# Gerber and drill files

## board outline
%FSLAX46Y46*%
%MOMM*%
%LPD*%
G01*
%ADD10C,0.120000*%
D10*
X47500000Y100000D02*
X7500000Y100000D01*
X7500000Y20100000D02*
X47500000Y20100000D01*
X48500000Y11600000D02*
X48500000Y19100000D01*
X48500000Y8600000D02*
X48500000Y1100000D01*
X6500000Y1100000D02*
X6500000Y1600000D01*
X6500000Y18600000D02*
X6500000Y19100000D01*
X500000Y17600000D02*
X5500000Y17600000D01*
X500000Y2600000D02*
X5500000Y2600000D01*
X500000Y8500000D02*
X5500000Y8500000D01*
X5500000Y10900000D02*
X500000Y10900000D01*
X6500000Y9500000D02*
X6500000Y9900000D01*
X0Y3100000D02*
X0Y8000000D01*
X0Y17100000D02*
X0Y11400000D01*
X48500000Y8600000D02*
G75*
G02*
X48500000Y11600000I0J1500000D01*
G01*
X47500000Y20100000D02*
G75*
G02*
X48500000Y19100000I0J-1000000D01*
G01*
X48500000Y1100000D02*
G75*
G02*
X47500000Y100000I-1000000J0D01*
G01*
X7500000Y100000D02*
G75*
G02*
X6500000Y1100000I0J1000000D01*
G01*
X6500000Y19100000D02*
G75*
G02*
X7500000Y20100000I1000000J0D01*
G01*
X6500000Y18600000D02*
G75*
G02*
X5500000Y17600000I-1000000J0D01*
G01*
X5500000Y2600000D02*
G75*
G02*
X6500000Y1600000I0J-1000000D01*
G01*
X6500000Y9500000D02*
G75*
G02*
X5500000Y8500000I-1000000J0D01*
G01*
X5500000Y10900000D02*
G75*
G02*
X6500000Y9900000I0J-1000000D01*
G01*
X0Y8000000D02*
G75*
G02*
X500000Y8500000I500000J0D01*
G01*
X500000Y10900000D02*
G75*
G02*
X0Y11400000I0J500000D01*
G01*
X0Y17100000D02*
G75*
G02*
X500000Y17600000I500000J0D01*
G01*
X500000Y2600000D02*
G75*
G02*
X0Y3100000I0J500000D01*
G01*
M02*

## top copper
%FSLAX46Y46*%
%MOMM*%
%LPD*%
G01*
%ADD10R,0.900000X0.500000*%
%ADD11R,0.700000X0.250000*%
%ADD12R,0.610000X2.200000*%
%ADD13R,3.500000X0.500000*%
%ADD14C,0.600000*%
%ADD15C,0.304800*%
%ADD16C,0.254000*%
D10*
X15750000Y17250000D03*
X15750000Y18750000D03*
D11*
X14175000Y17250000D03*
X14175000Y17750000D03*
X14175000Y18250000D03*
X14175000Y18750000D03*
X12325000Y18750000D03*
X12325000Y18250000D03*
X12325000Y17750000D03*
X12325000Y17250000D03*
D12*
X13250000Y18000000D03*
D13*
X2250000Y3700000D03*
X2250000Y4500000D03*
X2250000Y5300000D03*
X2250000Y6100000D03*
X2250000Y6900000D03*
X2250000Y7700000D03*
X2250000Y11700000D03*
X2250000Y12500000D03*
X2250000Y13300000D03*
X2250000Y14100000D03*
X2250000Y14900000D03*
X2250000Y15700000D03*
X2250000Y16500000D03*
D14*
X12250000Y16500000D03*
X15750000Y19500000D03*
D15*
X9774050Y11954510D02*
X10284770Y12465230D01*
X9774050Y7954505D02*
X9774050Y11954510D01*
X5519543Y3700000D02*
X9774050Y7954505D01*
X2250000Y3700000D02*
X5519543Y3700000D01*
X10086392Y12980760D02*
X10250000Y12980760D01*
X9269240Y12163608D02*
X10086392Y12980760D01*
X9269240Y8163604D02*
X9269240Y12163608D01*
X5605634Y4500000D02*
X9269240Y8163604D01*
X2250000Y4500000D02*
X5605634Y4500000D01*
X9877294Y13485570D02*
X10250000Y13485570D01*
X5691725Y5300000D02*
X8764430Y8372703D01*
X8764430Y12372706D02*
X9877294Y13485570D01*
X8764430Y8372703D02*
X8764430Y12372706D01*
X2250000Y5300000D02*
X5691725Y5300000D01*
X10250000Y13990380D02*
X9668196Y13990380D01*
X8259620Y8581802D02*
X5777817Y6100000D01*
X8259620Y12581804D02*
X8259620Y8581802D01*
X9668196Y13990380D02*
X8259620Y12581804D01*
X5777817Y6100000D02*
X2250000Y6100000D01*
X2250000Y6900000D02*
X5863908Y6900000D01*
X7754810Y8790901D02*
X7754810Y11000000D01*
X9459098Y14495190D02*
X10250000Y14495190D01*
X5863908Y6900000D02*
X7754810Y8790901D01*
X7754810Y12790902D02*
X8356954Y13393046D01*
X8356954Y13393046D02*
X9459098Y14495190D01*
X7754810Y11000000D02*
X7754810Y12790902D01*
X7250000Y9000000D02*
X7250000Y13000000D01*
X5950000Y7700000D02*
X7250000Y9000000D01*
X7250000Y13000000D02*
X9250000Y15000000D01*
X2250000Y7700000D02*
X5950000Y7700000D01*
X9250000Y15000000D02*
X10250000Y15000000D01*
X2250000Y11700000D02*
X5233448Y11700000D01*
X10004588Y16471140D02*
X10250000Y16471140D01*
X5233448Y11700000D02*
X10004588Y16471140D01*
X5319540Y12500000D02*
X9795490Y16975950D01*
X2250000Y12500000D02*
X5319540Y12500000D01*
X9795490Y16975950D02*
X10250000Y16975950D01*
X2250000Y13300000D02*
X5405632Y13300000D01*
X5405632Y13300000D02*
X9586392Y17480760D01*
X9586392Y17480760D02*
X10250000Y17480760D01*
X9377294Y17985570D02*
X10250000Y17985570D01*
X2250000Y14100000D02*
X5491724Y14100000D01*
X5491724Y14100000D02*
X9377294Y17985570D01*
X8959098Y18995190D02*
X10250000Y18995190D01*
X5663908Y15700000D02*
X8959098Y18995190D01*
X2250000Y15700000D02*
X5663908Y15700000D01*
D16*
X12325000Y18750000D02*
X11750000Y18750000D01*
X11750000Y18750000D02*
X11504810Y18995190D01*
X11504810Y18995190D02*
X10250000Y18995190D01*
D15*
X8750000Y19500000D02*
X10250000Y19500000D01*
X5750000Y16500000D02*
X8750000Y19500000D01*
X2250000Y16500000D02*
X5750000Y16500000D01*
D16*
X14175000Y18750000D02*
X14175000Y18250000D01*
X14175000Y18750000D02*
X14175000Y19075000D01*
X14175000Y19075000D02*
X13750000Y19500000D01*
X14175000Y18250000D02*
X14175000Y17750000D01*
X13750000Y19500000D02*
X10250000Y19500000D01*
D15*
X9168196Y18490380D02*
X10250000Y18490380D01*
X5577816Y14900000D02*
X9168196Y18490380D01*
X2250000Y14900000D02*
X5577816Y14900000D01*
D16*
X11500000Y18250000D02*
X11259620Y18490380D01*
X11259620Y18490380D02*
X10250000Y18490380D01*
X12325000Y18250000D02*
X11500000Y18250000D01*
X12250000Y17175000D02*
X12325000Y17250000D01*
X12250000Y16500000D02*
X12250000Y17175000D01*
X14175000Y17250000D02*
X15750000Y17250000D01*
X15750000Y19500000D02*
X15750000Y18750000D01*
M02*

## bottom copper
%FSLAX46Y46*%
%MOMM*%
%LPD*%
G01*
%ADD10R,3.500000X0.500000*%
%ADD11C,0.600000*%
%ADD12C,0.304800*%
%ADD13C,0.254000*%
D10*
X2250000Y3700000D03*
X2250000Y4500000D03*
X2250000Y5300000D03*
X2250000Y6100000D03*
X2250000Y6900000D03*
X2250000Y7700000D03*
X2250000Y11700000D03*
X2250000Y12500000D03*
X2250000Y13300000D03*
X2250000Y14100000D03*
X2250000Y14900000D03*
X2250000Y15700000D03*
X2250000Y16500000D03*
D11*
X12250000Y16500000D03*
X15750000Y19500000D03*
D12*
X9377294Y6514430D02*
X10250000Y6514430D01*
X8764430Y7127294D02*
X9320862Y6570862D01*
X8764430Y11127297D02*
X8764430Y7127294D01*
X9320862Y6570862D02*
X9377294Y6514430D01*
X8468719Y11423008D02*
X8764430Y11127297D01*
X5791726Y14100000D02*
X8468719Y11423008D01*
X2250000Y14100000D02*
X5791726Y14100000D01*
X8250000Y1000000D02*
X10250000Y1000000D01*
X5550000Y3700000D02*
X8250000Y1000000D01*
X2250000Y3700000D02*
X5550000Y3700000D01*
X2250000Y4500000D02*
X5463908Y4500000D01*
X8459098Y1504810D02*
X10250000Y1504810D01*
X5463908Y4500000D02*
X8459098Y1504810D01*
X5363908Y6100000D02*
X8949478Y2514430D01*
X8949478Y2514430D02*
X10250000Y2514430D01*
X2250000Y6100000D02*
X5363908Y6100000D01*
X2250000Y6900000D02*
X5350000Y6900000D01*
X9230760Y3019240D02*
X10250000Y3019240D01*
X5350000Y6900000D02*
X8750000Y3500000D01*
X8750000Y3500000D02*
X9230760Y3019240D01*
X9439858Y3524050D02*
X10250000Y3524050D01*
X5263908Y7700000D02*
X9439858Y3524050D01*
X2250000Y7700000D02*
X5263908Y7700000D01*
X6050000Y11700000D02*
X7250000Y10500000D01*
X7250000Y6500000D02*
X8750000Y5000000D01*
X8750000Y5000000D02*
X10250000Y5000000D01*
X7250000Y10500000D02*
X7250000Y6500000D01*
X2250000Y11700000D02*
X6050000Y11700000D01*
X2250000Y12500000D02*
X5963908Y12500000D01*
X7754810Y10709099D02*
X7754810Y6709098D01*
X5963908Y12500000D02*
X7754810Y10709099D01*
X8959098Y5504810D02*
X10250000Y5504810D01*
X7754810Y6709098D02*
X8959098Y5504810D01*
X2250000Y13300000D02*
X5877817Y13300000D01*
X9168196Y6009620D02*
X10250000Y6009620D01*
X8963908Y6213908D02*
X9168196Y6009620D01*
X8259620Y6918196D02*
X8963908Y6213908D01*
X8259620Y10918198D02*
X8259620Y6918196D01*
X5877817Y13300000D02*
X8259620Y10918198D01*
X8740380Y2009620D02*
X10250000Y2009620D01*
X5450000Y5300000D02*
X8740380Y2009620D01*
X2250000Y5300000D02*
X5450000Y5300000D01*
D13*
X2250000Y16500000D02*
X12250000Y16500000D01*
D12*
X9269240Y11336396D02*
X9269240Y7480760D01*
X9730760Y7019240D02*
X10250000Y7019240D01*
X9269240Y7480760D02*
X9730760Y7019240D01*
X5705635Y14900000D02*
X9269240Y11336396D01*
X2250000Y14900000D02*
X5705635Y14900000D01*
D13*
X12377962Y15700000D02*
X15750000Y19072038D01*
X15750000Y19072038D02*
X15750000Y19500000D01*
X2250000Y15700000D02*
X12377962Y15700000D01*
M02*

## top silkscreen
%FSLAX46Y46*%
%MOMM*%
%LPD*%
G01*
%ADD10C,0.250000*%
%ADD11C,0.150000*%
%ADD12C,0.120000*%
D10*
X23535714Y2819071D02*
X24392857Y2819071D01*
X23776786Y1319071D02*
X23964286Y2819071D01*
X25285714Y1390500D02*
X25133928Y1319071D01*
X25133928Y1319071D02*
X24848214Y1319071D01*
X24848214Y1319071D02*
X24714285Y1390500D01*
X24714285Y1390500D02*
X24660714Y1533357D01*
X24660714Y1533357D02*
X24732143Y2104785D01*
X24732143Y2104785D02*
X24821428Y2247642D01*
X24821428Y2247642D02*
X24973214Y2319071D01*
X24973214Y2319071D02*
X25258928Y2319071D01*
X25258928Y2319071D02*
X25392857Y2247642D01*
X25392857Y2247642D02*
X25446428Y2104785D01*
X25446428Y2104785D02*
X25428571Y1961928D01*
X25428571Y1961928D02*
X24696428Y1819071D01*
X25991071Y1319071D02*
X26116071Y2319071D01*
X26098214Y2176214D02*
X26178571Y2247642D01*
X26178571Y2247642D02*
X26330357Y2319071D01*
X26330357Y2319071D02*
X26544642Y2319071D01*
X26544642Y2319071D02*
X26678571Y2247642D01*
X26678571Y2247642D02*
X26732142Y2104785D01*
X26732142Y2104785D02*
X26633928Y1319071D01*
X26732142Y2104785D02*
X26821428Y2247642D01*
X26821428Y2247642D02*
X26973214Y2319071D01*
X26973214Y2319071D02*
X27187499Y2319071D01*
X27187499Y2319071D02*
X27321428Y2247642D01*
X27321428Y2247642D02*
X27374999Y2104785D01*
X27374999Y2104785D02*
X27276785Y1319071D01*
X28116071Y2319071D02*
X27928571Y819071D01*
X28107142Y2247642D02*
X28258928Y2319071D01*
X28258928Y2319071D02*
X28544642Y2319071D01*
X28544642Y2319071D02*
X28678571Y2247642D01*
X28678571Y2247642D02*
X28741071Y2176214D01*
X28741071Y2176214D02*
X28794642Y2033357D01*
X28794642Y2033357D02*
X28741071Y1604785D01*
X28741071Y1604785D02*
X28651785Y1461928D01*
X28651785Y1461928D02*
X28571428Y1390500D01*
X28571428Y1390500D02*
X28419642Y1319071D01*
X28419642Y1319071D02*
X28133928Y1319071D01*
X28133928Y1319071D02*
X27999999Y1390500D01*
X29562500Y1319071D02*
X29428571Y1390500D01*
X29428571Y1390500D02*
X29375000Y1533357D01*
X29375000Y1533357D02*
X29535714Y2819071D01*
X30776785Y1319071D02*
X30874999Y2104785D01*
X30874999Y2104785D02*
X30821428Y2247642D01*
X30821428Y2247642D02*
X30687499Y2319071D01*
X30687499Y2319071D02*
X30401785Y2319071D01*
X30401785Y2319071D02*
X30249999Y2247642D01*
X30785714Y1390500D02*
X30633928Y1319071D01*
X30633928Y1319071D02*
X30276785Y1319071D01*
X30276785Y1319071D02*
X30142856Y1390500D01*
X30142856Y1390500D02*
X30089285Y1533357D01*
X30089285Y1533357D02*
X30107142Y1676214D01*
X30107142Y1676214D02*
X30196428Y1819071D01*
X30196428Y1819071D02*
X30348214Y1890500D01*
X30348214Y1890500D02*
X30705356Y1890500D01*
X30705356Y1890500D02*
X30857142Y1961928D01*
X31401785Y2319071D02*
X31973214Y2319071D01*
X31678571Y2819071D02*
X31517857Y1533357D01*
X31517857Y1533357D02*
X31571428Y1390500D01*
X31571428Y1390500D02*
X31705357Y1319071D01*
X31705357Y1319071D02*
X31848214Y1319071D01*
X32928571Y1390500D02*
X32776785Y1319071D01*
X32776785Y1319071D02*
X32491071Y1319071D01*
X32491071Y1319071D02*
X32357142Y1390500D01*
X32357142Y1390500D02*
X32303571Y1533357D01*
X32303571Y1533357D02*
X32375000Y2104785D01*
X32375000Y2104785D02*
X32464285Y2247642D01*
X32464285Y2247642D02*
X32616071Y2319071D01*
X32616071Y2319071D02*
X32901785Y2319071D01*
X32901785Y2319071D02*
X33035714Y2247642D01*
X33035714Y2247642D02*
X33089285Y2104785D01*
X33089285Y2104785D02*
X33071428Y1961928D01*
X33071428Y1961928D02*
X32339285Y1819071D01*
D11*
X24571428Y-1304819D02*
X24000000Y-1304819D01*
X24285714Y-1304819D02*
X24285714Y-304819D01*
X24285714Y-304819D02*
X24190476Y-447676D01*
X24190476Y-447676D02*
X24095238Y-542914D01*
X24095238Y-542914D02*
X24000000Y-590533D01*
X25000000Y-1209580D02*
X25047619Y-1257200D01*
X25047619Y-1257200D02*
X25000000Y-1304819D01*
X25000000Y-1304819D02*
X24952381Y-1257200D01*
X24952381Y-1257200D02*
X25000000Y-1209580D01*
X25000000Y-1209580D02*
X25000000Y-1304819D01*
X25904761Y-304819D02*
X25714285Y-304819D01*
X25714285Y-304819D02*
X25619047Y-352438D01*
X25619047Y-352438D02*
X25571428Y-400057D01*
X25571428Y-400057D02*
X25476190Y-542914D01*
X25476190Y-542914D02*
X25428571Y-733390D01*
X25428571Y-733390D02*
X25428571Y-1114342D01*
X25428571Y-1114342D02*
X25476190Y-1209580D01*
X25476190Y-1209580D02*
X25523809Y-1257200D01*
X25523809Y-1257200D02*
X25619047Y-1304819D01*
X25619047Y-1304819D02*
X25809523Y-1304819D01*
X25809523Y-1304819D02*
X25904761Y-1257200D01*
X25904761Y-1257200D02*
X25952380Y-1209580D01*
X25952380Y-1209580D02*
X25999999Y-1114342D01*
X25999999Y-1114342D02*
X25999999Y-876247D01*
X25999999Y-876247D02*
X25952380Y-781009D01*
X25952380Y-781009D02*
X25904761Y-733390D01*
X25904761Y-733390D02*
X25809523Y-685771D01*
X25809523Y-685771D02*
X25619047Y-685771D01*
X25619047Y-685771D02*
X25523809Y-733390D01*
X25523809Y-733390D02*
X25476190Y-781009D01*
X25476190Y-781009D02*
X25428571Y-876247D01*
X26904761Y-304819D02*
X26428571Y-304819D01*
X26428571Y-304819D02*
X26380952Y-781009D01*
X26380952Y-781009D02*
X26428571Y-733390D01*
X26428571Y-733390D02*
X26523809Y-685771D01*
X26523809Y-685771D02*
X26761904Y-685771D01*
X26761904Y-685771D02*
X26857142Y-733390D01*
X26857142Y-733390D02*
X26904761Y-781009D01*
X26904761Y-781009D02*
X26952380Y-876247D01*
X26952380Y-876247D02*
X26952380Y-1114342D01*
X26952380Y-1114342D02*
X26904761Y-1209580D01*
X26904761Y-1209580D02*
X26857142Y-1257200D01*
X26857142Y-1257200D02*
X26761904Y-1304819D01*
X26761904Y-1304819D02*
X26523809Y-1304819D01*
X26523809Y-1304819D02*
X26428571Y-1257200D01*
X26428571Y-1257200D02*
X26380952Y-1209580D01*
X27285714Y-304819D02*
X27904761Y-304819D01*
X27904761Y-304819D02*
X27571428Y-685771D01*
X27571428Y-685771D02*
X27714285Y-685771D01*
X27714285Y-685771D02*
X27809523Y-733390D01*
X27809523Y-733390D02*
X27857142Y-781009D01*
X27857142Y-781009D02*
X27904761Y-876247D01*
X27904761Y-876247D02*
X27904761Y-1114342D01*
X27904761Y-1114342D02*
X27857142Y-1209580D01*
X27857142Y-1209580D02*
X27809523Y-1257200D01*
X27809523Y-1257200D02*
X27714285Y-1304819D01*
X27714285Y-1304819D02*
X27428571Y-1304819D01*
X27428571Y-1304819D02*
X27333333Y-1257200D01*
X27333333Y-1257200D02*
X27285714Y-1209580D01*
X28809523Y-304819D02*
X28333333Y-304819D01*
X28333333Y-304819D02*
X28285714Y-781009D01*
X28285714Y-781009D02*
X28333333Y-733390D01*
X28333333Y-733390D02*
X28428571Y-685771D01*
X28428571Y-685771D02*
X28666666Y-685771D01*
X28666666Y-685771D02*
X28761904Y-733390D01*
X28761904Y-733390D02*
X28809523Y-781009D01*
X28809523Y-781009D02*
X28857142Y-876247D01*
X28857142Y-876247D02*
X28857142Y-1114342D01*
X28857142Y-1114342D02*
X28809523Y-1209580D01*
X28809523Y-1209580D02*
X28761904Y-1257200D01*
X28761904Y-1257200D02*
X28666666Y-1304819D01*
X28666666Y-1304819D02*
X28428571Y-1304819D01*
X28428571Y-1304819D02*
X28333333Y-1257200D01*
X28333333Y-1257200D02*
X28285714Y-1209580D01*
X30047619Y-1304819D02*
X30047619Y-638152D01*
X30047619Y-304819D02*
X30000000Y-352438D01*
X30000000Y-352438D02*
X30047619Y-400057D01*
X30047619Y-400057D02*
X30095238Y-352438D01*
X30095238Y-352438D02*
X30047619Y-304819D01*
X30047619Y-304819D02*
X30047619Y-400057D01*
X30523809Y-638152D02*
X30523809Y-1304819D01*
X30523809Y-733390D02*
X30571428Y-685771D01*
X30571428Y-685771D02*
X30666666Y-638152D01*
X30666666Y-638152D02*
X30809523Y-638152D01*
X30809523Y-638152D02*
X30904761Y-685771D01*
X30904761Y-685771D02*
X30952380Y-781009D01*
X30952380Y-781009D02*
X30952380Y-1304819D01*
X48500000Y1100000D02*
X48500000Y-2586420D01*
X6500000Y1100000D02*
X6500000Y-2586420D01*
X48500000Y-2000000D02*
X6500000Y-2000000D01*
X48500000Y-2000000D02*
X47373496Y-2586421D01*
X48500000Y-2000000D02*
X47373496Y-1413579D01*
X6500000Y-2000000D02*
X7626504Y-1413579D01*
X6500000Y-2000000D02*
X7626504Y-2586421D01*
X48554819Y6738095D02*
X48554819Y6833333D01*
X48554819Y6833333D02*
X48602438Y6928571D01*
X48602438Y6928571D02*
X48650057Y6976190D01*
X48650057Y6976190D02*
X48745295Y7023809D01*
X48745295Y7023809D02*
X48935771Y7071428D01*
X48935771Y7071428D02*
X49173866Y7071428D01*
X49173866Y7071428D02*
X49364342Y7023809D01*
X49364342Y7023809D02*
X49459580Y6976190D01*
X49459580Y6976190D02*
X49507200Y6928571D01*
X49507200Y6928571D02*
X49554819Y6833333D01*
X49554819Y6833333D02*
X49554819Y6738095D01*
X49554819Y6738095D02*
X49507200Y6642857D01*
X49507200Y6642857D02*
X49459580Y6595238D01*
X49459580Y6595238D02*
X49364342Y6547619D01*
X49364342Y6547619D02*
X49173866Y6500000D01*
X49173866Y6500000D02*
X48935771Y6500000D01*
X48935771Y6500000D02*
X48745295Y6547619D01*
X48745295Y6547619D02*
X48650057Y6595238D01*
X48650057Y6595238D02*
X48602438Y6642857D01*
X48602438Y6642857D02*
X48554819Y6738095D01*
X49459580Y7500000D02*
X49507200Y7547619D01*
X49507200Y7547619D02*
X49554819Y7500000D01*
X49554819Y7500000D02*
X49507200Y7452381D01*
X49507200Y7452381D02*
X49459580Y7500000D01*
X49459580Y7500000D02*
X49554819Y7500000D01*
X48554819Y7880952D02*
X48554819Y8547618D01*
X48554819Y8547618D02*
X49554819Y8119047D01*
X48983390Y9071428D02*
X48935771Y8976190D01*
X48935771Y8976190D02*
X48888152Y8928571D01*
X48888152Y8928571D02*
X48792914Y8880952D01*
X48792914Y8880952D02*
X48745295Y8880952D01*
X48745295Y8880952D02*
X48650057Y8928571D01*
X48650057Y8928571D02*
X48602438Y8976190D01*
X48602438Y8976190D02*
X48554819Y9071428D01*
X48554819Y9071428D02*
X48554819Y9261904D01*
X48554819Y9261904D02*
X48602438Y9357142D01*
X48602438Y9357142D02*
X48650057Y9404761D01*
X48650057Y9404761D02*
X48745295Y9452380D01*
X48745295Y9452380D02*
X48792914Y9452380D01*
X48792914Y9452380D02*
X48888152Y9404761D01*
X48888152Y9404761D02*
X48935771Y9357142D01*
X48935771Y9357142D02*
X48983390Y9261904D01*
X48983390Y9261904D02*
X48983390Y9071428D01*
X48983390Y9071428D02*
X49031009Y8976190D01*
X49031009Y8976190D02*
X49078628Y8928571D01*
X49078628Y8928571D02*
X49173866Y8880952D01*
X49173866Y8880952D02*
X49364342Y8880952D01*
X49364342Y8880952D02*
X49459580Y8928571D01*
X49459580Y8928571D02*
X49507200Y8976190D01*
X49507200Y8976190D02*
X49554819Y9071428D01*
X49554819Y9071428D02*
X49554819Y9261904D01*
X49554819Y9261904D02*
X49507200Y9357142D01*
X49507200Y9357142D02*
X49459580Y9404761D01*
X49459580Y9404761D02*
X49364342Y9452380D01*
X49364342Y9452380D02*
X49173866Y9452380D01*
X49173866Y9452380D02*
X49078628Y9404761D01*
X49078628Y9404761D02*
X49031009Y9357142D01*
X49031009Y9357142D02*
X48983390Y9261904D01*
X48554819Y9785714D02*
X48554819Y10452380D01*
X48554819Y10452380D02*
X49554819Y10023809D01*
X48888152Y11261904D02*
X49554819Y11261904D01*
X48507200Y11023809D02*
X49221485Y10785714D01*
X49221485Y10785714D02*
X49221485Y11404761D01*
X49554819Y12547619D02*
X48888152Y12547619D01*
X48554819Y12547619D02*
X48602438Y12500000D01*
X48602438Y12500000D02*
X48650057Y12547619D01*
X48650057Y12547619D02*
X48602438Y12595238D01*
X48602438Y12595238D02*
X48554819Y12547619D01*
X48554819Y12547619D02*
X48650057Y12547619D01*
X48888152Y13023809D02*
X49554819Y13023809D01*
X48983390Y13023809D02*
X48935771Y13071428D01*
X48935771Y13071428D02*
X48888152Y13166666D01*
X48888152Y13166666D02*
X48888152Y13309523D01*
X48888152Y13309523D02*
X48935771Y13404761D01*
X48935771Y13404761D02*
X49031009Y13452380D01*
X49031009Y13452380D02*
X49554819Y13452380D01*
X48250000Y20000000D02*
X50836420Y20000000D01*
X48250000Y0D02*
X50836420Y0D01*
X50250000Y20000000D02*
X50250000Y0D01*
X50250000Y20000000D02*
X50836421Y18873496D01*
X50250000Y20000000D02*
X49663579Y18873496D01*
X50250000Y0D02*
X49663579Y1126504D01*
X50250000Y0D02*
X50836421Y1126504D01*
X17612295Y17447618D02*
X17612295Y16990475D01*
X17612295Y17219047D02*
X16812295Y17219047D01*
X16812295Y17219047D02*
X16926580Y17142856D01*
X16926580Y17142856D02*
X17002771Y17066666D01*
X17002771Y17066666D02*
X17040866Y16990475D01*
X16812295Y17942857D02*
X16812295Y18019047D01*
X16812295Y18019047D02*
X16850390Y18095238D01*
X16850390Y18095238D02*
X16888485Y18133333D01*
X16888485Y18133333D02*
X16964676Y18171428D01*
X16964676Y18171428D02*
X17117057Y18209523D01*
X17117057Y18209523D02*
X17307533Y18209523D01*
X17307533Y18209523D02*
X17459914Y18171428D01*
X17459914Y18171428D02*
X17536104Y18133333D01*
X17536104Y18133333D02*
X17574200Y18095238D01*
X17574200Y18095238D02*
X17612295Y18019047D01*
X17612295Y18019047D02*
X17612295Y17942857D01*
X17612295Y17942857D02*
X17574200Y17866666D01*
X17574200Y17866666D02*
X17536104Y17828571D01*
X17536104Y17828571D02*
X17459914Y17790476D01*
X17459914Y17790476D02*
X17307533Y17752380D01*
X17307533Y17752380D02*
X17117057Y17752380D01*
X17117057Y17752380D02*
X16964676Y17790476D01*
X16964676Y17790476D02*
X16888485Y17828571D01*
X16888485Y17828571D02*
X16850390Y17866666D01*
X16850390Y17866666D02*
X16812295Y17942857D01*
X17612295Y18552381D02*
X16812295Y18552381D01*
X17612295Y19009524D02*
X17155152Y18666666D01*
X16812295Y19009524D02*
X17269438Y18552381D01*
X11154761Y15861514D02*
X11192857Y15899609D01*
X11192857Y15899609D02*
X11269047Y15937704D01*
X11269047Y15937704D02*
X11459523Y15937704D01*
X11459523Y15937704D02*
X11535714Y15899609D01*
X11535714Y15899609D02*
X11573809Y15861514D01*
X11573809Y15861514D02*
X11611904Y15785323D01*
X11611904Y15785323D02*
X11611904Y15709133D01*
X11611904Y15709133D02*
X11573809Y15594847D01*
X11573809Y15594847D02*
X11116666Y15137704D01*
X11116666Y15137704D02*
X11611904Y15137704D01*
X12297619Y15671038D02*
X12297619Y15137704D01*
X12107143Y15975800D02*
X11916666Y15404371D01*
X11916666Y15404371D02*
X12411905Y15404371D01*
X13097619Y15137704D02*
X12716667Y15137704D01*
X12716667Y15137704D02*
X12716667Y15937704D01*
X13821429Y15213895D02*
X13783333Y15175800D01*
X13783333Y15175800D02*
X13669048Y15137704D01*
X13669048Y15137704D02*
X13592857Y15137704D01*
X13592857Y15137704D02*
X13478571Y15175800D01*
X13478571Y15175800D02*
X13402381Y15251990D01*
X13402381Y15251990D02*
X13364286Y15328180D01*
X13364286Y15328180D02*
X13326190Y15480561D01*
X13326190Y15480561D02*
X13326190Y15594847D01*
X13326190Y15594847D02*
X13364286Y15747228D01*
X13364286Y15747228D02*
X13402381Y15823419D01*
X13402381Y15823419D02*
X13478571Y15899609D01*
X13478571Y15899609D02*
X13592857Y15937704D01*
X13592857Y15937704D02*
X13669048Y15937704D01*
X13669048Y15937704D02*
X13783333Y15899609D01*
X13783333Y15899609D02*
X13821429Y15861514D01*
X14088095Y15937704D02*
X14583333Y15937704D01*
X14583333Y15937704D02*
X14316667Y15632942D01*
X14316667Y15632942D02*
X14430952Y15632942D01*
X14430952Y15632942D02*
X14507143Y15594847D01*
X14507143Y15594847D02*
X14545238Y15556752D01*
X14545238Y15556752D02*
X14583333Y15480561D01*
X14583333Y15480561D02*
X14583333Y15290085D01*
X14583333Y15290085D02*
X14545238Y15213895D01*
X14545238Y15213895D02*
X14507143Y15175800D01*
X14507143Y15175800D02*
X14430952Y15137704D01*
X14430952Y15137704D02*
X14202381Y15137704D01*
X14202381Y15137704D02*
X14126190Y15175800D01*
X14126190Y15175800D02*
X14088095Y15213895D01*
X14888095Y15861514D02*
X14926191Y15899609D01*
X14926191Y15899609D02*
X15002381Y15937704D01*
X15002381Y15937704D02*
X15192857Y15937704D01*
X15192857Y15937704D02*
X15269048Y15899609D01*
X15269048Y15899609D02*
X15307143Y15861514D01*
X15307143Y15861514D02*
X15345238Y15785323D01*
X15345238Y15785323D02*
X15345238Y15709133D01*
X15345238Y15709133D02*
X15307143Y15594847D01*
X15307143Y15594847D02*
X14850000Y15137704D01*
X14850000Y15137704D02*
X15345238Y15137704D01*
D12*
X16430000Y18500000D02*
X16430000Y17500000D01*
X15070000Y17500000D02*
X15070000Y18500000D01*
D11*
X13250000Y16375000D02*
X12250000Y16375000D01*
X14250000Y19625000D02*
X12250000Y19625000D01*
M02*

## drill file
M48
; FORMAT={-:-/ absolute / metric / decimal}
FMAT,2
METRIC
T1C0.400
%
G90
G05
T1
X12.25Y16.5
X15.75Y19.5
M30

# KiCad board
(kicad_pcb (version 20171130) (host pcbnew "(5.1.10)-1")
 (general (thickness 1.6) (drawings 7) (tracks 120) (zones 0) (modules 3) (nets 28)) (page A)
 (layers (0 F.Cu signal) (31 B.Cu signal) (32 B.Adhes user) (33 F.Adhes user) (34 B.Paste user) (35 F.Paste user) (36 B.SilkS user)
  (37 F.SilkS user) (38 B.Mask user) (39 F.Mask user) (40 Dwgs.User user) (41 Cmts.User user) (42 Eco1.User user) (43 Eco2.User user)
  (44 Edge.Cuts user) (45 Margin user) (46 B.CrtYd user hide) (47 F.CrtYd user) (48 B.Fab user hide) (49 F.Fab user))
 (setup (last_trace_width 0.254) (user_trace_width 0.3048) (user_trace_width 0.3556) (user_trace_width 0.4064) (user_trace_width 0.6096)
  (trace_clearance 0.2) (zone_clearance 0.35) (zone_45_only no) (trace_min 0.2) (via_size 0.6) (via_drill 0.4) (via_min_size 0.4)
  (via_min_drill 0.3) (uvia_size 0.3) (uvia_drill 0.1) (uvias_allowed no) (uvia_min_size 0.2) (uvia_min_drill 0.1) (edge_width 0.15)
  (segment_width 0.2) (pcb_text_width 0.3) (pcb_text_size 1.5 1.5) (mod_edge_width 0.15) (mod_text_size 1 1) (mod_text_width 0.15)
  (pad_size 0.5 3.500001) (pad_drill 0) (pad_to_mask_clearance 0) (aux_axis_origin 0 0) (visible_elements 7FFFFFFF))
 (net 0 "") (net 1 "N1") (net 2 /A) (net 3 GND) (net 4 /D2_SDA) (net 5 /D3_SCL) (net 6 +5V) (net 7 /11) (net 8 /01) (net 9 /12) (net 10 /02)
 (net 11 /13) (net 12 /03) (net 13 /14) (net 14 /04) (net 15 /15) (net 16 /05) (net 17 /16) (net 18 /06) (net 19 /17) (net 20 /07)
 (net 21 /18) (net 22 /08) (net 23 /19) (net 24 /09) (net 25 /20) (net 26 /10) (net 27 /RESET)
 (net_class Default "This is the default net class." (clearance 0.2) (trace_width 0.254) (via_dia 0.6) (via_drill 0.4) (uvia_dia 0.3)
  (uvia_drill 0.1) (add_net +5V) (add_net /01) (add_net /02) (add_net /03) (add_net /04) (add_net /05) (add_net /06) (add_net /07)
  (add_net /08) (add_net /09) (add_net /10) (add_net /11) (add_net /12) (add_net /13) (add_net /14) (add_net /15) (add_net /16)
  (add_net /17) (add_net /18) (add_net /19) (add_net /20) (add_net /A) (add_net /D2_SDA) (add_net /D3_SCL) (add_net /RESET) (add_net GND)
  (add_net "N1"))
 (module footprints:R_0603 (layer F.Cu) (at 15.75 -18 90)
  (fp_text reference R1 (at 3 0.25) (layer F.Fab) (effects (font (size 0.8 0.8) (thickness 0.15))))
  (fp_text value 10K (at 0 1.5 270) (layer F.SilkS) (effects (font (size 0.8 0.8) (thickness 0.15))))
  (fp_line (start 0.5 0.68) (end -0.5 0.68) (layer F.SilkS) (width 0.12))
  (fp_line (start -0.5 -0.68) (end 0.5 -0.68) (layer F.SilkS) (width 0.12))
  (pad 1 smd rect (at -0.75 0 90) (size 0.5 0.9) (layers F.Cu F.Paste F.Mask) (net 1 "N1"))
  (pad 2 smd rect (at 0.75 0 90) (size 0.5 0.9) (layers F.Cu F.Paste F.Mask) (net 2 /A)))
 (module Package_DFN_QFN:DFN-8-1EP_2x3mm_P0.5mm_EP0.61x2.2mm (layer F.Cu) (at 13.25 -18 180)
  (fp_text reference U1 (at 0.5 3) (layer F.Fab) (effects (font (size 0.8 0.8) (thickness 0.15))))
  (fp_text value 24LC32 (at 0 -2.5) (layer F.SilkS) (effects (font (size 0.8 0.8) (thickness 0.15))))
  (fp_line (start 0 -1.625) (end 1 -1.625) (layer F.SilkS) (width 0.15))
  (fp_line (start -1 1.625) (end 1 1.625) (layer F.SilkS) (width 0.15))
  (pad 1 smd rect (at -0.925 -0.75 180) (size 0.7 0.25) (layers F.Cu F.Paste F.Mask) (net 1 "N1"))
  (pad 2 smd rect (at -0.925 -0.25 180) (size 0.7 0.25) (layers F.Cu F.Paste F.Mask) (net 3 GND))
  (pad 3 smd rect (at -0.925 0.25 180) (size 0.7 0.25) (layers F.Cu F.Paste F.Mask) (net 3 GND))
  (pad 4 smd rect (at -0.925 0.75 180) (size 0.7 0.25) (layers F.Cu F.Paste F.Mask) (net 3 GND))
  (pad 5 smd rect (at 0.925 0.75 180) (size 0.7 0.25) (layers F.Cu F.Paste F.Mask) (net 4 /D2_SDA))
  (pad 6 smd rect (at 0.925 0.25 180) (size 0.7 0.25) (layers F.Cu F.Paste F.Mask) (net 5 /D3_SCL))
  (pad 7 smd rect (at 0.925 -0.25 180) (size 0.7 0.25) (layers F.Cu F.Paste F.Mask))
  (pad 8 smd rect (at 0.925 -0.75 180) (size 0.7 0.25) (layers F.Cu F.Paste F.Mask) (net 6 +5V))
  (pad 9 smd rect (at 0 0 180) (size 0.61 2.2) (layers F.Cu F.Mask))
  (pad "" smd rect (at 0 -0.734 180) (size 0.5 0.59) (layers F.Paste))
  (pad "" smd rect (at 0 0 180) (size 0.5 0.59) (layers F.Paste))
  (pad "" smd rect (at 0 0.734 180) (size 0.5 0.59) (layers F.Paste)))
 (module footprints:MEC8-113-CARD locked (layer F.Cu) (at 0 -0.1 90)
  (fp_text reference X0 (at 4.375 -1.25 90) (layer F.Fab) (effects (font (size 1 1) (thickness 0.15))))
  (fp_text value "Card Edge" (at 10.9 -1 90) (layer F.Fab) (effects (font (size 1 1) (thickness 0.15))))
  (fp_line (start 0 47.5) (end 0 7.5) (layer Edge.Cuts) (width 0.12))
  (fp_line (start 20 7.5) (end 20 47.5) (layer Edge.Cuts) (width 0.12))
  (fp_line (start 11.5 48.5) (end 19 48.5) (layer Edge.Cuts) (width 0.12))
  (fp_line (start 8.5 48.5) (end 1 48.5) (layer Edge.Cuts) (width 0.12))
  (fp_line (start 1 6.5) (end 1.5 6.5) (layer Edge.Cuts) (width 0.12))
  (fp_line (start 18.5 6.5) (end 19 6.5) (layer Edge.Cuts) (width 0.12))
  (fp_line (start 17.5 0.5) (end 17.5 5.5) (layer Edge.Cuts) (width 0.12))
  (fp_line (start 2.5 0.5) (end 2.5 5.5) (layer Edge.Cuts) (width 0.12))
  (fp_line (start 8.4 0.5) (end 8.4 5.5) (layer Edge.Cuts) (width 0.12))
  (fp_line (start 10.8 5.5) (end 10.8 0.5) (layer Edge.Cuts) (width 0.12))
  (fp_line (start 9.4 6.5) (end 9.8 6.5) (layer Edge.Cuts) (width 0.12))
  (fp_line (start 3 0) (end 7.9 0) (layer Edge.Cuts) (width 0.12))
  (fp_line (start 17 0) (end 11.3 0) (layer Edge.Cuts) (width 0.12))
  (fp_arc (start 10 48.5) (end 11.5 48.5) (angle -180) (layer Edge.Cuts) (width 0.12))
  (fp_arc (start 19 47.5) (end 19 48.5) (angle -90) (layer Edge.Cuts) (width 0.12))
  (fp_arc (start 1 47.5) (end 0 47.5) (angle -90) (layer Edge.Cuts) (width 0.12))
  (fp_arc (start 1 7.5) (end 1 6.5) (angle -90) (layer Edge.Cuts) (width 0.12))
  (fp_arc (start 19 7.5) (end 20 7.5) (angle -90) (layer Edge.Cuts) (width 0.12))
  (fp_arc (start 18.5 5.5) (end 17.5 5.5) (angle -90) (layer Edge.Cuts) (width 0.12))
  (fp_arc (start 1.5 5.5) (end 1.5 6.5) (angle -90) (layer Edge.Cuts) (width 0.12))
  (fp_arc (start 9.4 5.5) (end 8.4 5.5) (angle -90) (layer Edge.Cuts) (width 0.12))
  (fp_arc (start 9.8 5.5) (end 9.8 6.5) (angle -90) (layer Edge.Cuts) (width 0.12))
  (fp_arc (start 7.9 0.5) (end 8.4 0.5) (angle -90) (layer Edge.Cuts) (width 0.12))
  (fp_arc (start 11.3 0.5) (end 11.3 0) (angle -90) (layer Edge.Cuts) (width 0.12))
  (fp_arc (start 17 0.5) (end 17.5 0.5) (angle -90) (layer Edge.Cuts) (width 0.12))
  (fp_arc (start 3 0.5) (end 3 0) (angle -90) (layer Edge.Cuts) (width 0.12))
  (pad 14 smd rect (at 3.6 2.25 90) (size 0.5 3.5) (layers F.Cu F.Paste F.Mask) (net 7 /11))
  (pad 1 smd rect (at 3.6 2.25 90) (size 0.5 3.5) (layers B.Cu B.Paste B.Mask) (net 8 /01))
  (pad 15 smd rect (at 4.4 2.25 90) (size 0.5 3.5) (layers F.Cu F.Paste F.Mask) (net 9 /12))
  (pad 2 smd rect (at 4.4 2.25 90) (size 0.5 3.5) (layers B.Cu B.Paste B.Mask) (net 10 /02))
  (pad 16 smd rect (at 5.2 2.25 90) (size 0.5 3.5) (layers F.Cu F.Paste F.Mask) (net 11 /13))
  (pad 3 smd rect (at 5.2 2.25 90) (size 0.5 3.5) (layers B.Cu B.Paste B.Mask) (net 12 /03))
  (pad 17 smd rect (at 6 2.25 90) (size 0.5 3.5) (layers F.Cu F.Paste F.Mask) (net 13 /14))
  (pad 4 smd rect (at 6 2.25 90) (size 0.5 3.5) (layers B.Cu B.Paste B.Mask) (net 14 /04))
  (pad 18 smd rect (at 6.8 2.25 90) (size 0.5 3.5) (layers F.Cu F.Paste F.Mask) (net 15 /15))
  (pad 5 smd rect (at 6.8 2.25 90) (size 0.5 3.5) (layers B.Cu B.Paste B.Mask) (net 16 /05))
  (pad 19 smd rect (at 7.6 2.25 90) (size 0.5 3.5) (layers F.Cu F.Paste F.Mask) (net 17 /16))
  (pad 6 smd rect (at 7.6 2.25 90) (size 0.5 3.5) (layers B.Cu B.Paste B.Mask) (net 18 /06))
  (pad 20 smd rect (at 11.6 2.25 90) (size 0.5 3.5) (layers F.Cu F.Paste F.Mask) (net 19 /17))
  (pad 7 smd rect (at 11.6 2.25 90) (size 0.5 3.5) (layers B.Cu B.Paste B.Mask) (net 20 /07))
  (pad 21 smd rect (at 12.4 2.25 90) (size 0.5 3.5) (layers F.Cu F.Paste F.Mask) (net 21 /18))
  (pad 8 smd rect (at 12.4 2.25 90) (size 0.5 3.5) (layers B.Cu B.Paste B.Mask) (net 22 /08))
  (pad 22 smd rect (at 13.2 2.25 90) (size 0.5 3.5) (layers F.Cu F.Paste F.Mask) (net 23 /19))
  (pad 9 smd rect (at 13.2 2.25 90) (size 0.5 3.5) (layers B.Cu B.Paste B.Mask) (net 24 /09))
  (pad 23 smd rect (at 14 2.25 90) (size 0.5 3.5) (layers F.Cu F.Paste F.Mask) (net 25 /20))
  (pad 10 smd rect (at 14 2.25 90) (size 0.5 3.5) (layers B.Cu B.Paste B.Mask) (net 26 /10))
  (pad 24 smd rect (at 14.8 2.25 90) (size 0.5 3.5) (layers F.Cu F.Paste F.Mask) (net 5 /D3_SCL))
  (pad 11 smd rect (at 14.8 2.25 90) (size 0.5 3.5) (layers B.Cu B.Paste B.Mask) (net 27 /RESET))
  (pad 25 smd rect (at 15.6 2.25 90) (size 0.5 3.5) (layers F.Cu F.Paste F.Mask) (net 4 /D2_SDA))
  (pad 12 smd rect (at 15.6 2.25 90) (size 0.5 3.5) (layers B.Cu B.Paste B.Mask) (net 2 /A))
  (pad 26 smd rect (at 16.4 2.25 90) (size 0.5 3.5) (layers F.Cu F.Paste F.Mask) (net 3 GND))
  (pad 13 smd rect (at 16.4 2.25 90) (size 0.5 3.5) (layers B.Cu B.Paste B.Mask) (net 6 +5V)))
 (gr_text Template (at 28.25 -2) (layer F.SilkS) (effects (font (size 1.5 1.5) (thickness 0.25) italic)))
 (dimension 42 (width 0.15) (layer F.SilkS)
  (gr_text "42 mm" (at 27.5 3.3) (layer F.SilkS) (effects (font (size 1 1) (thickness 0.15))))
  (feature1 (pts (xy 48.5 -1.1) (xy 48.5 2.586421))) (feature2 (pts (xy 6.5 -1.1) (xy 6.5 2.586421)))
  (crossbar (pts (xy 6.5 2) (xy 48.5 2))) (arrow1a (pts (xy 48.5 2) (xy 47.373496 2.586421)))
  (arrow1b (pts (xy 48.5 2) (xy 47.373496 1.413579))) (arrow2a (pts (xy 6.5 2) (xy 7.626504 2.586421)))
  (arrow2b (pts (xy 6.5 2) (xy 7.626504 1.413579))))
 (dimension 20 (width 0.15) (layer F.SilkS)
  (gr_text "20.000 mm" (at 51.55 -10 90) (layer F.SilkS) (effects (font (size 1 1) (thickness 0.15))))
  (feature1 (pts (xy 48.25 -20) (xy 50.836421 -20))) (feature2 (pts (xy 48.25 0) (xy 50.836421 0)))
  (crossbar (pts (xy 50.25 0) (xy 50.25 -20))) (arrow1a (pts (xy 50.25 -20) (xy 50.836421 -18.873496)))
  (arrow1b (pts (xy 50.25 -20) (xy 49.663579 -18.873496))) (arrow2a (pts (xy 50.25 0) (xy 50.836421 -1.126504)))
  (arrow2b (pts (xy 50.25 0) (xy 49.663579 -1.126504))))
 (segment (start 9.377294 -6.51443) (end 10.25 -6.51443) (width 0.3048) (layer B.Cu) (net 26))
 (segment (start 8.76443 -7.127294) (end 9.320862 -6.570862) (width 0.3048) (layer B.Cu) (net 26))
 (segment (start 8.76443 -11.127297) (end 8.76443 -7.127294) (width 0.3048) (layer B.Cu) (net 26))
 (segment (start 9.320862 -6.570862) (end 9.377294 -6.51443) (width 0.3048) (layer B.Cu) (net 26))
 (segment (start 8.468719 -11.423008) (end 8.76443 -11.127297) (width 0.3048) (layer B.Cu) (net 26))
 (segment (start 5.791726 -14.1) (end 8.468719 -11.423008) (width 0.3048) (layer B.Cu) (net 26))
 (segment (start 2.25 -14.1) (end 5.791726 -14.1) (width 0.3048) (layer B.Cu) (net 26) (status 10))
 (segment (start 8.25 -1) (end 10.25 -1) (width 0.3048) (layer B.Cu) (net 8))
 (segment (start 5.55 -3.7) (end 8.25 -1) (width 0.3048) (layer B.Cu) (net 8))
 (segment (start 2.25 -3.7) (end 5.55 -3.7) (width 0.3048) (layer B.Cu) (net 8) (status 10))
 (segment (start 2.25 -4.5) (end 5.463908 -4.5) (width 0.3048) (layer B.Cu) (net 10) (status 10))
 (segment (start 8.459098 -1.50481) (end 10.25 -1.50481) (width 0.3048) (layer B.Cu) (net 10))
 (segment (start 5.463908 -4.5) (end 8.459098 -1.50481) (width 0.3048) (layer B.Cu) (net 10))
 (segment (start 5.363908 -6.1) (end 8.949478 -2.51443) (width 0.3048) (layer B.Cu) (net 14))
 (segment (start 8.949478 -2.51443) (end 10.25 -2.51443) (width 0.3048) (layer B.Cu) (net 14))
 (segment (start 2.25 -6.1) (end 5.363908 -6.1) (width 0.3048) (layer B.Cu) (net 14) (status 10))
 (segment (start 2.25 -6.9) (end 5.35 -6.9) (width 0.3048) (layer B.Cu) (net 16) (status 10))
 (segment (start 9.23076 -3.01924) (end 10.25 -3.01924) (width 0.3048) (layer B.Cu) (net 16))
 (segment (start 5.35 -6.9) (end 8.75 -3.5) (width 0.3048) (layer B.Cu) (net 16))
 (segment (start 8.75 -3.5) (end 9.23076 -3.01924) (width 0.3048) (layer B.Cu) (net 16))
 (segment (start 9.439858 -3.52405) (end 10.25 -3.52405) (width 0.3048) (layer B.Cu) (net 18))
 (segment (start 5.263908 -7.7) (end 9.439858 -3.52405) (width 0.3048) (layer B.Cu) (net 18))
 (segment (start 2.25 -7.7) (end 5.263908 -7.7) (width 0.3048) (layer B.Cu) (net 18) (status 10))
 (segment (start 6.05 -11.7) (end 7.25 -10.5) (width 0.3048) (layer B.Cu) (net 20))
 (segment (start 7.25 -6.5) (end 8.75 -5) (width 0.3048) (layer B.Cu) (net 20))
 (segment (start 8.75 -5) (end 10.25 -5) (width 0.3048) (layer B.Cu) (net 20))
 (segment (start 7.25 -10.5) (end 7.25 -6.5) (width 0.3048) (layer B.Cu) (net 20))
 (segment (start 2.25 -11.7) (end 6.05 -11.7) (width 0.3048) (layer B.Cu) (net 20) (status 10))
 (segment (start 2.25 -12.5) (end 5.963908 -12.5) (width 0.3048) (layer B.Cu) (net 22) (status 10))
 (segment (start 7.75481 -10.709099) (end 7.75481 -6.709098) (width 0.3048) (layer B.Cu) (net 22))
 (segment (start 5.963908 -12.5) (end 7.75481 -10.709099) (width 0.3048) (layer B.Cu) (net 22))
 (segment (start 8.959098 -5.50481) (end 10.25 -5.50481) (width 0.3048) (layer B.Cu) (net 22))
 (segment (start 7.75481 -6.709098) (end 8.959098 -5.50481) (width 0.3048) (layer B.Cu) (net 22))
 (segment (start 2.25 -13.3) (end 5.877817 -13.3) (width 0.3048) (layer B.Cu) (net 24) (status 10))
 (segment (start 9.168196 -6.00962) (end 10.25 -6.00962) (width 0.3048) (layer B.Cu) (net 24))
 (segment (start 8.963908 -6.213908) (end 9.168196 -6.00962) (width 0.3048) (layer B.Cu) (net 24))
 (segment (start 8.25962 -6.918196) (end 8.963908 -6.213908) (width 0.3048) (layer B.Cu) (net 24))
 (segment (start 8.25962 -10.918198) (end 8.25962 -6.918196) (width 0.3048) (layer B.Cu) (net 24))
 (segment (start 5.877817 -13.3) (end 8.25962 -10.918198) (width 0.3048) (layer B.Cu) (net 24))
 (segment (start 9.77405 -11.95451) (end 10.28477 -12.46523) (width 0.3048) (layer F.Cu) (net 7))
 (segment (start 9.77405 -7.954505) (end 9.77405 -11.95451) (width 0.3048) (layer F.Cu) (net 7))
 (segment (start 5.519543 -3.7) (end 9.77405 -7.954505) (width 0.3048) (layer F.Cu) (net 7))
 (segment (start 2.25 -3.7) (end 5.519543 -3.7) (width 0.3048) (layer F.Cu) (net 7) (status 10))
 (segment (start 10.086392 -12.98076) (end 10.25 -12.98076) (width 0.3048) (layer F.Cu) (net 9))
 (segment (start 9.26924 -12.163608) (end 10.086392 -12.98076) (width 0.3048) (layer F.Cu) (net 9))
 (segment (start 9.26924 -8.163604) (end 9.26924 -12.163608) (width 0.3048) (layer F.Cu) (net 9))
 (segment (start 5.605634 -4.5) (end 9.26924 -8.163604) (width 0.3048) (layer F.Cu) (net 9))
 (segment (start 2.25 -4.5) (end 5.605634 -4.5) (width 0.3048) (layer F.Cu) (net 9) (status 10))
 (segment (start 9.877294 -13.48557) (end 10.25 -13.48557) (width 0.3048) (layer F.Cu) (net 11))
 (segment (start 5.691725 -5.3) (end 8.76443 -8.372703) (width 0.3048) (layer F.Cu) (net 11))
 (segment (start 8.76443 -12.372706) (end 9.877294 -13.48557) (width 0.3048) (layer F.Cu) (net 11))
 (segment (start 8.76443 -8.372703) (end 8.76443 -12.372706) (width 0.3048) (layer F.Cu) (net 11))
 (segment (start 2.25 -5.3) (end 5.691725 -5.3) (width 0.3048) (layer F.Cu) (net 11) (status 10))
 (segment (start 10.25 -13.99038) (end 9.668196 -13.99038) (width 0.3048) (layer F.Cu) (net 13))
 (segment (start 8.25962 -8.581802) (end 5.777817 -6.1) (width 0.3048) (layer F.Cu) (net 13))
 (segment (start 8.25962 -12.581804) (end 8.25962 -8.581802) (width 0.3048) (layer F.Cu) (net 13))
 (segment (start 9.668196 -13.99038) (end 8.25962 -12.581804) (width 0.3048) (layer F.Cu) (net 13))
 (segment (start 5.777817 -6.1) (end 2.25 -6.1) (width 0.3048) (layer F.Cu) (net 13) (status 20))
 (segment (start 2.25 -6.9) (end 5.863908 -6.9) (width 0.3048) (layer F.Cu) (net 15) (status 10))
 (segment (start 7.75481 -8.790901) (end 7.75481 -11) (width 0.3048) (layer F.Cu) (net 15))
 (segment (start 9.459098 -14.49519) (end 10.25 -14.49519) (width 0.3048) (layer F.Cu) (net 15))
 (segment (start 5.863908 -6.9) (end 7.75481 -8.790901) (width 0.3048) (layer F.Cu) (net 15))
 (segment (start 7.75481 -12.790902) (end 8.356954 -13.393046) (width 0.3048) (layer F.Cu) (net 15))
 (segment (start 8.356954 -13.393046) (end 9.459098 -14.49519) (width 0.3048) (layer F.Cu) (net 15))
 (segment (start 7.75481 -11) (end 7.75481 -12.790902) (width 0.3048) (layer F.Cu) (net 15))
 (segment (start 7.25 -9) (end 7.25 -13) (width 0.3048) (layer F.Cu) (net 17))
 (segment (start 5.95 -7.7) (end 7.25 -9) (width 0.3048) (layer F.Cu) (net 17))
 (segment (start 7.25 -13) (end 9.25 -15) (width 0.3048) (layer F.Cu) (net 17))
 (segment (start 2.25 -7.7) (end 5.95 -7.7) (width 0.3048) (layer F.Cu) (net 17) (status 10))
 (segment (start 9.25 -15) (end 10.25 -15) (width 0.3048) (layer F.Cu) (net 17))
 (segment (start 2.25 -11.7) (end 5.233448 -11.7) (width 0.3048) (layer F.Cu) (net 19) (status 10))
 (segment (start 10.004588 -16.47114) (end 10.25 -16.47114) (width 0.3048) (layer F.Cu) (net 19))
 (segment (start 5.233448 -11.7) (end 10.004588 -16.47114) (width 0.3048) (layer F.Cu) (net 19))
 (segment (start 5.31954 -12.5) (end 9.79549 -16.97595) (width 0.3048) (layer F.Cu) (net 21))
 (segment (start 2.25 -12.5) (end 5.31954 -12.5) (width 0.3048) (layer F.Cu) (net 21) (status 10))
 (segment (start 9.79549 -16.97595) (end 10.25 -16.97595) (width 0.3048) (layer F.Cu) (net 21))
 (segment (start 2.25 -13.3) (end 5.405632 -13.3) (width 0.3048) (layer F.Cu) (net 23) (status 10))
 (segment (start 5.405632 -13.3) (end 9.586392 -17.48076) (width 0.3048) (layer F.Cu) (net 23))
 (segment (start 9.586392 -17.48076) (end 10.25 -17.48076) (width 0.3048) (layer F.Cu) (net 23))
 (segment (start 9.377294 -17.98557) (end 10.25 -17.98557) (width 0.3048) (layer F.Cu) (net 25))
 (segment (start 2.25 -14.1) (end 5.491724 -14.1) (width 0.3048) (layer F.Cu) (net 25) (status 10))
 (segment (start 5.491724 -14.1) (end 9.377294 -17.98557) (width 0.3048) (layer F.Cu) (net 25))
 (segment (start 8.74038 -2.00962) (end 10.25 -2.00962) (width 0.3048) (layer B.Cu) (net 12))
 (segment (start 5.45 -5.3) (end 8.74038 -2.00962) (width 0.3048) (layer B.Cu) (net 12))
 (segment (start 2.25 -5.3) (end 5.45 -5.3) (width 0.3048) (layer B.Cu) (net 12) (status 10))
 (segment (start 8.959098 -18.99519) (end 10.25 -18.99519) (width 0.3048) (layer F.Cu) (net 4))
 (segment (start 5.663908 -15.7) (end 8.959098 -18.99519) (width 0.3048) (layer F.Cu) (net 4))
 (segment (start 2.25 -15.7) (end 5.663908 -15.7) (width 0.3048) (layer F.Cu) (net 4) (status 10))
 (segment (start 12.325 -18.75) (end 11.75 -18.75) (width 0.254) (layer F.Cu) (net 4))
 (segment (start 11.75 -18.75) (end 11.50481 -18.99519) (width 0.254) (layer F.Cu) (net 4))
 (segment (start 11.50481 -18.99519) (end 10.25 -18.99519) (width 0.254) (layer F.Cu) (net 4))
 (segment (start 8.75 -19.5) (end 10.25 -19.5) (width 0.3048) (layer F.Cu) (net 3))
 (segment (start 5.75 -16.5) (end 8.75 -19.5) (width 0.3048) (layer F.Cu) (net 3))
 (segment (start 2.25 -16.5) (end 5.75 -16.5) (width 0.3048) (layer F.Cu) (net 3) (status 10))
 (segment (start 14.175 -18.75) (end 14.175 -18.25) (width 0.254) (layer F.Cu) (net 3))
 (segment (start 14.175 -18.75) (end 14.175 -19.075) (width 0.254) (layer F.Cu) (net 3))
 (segment (start 14.175 -19.075) (end 13.75 -19.5) (width 0.254) (layer F.Cu) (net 3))
 (segment (start 14.175 -18.25) (end 14.175 -17.75) (width 0.254) (layer F.Cu) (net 3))
 (segment (start 13.75 -19.5) (end 10.25 -19.5) (width 0.254) (layer F.Cu) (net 3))
 (segment (start 9.168196 -18.49038) (end 10.25 -18.49038) (width 0.3048) (layer F.Cu) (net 5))
 (segment (start 5.577816 -14.9) (end 9.168196 -18.49038) (width 0.3048) (layer F.Cu) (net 5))
 (segment (start 2.25 -14.9) (end 5.577816 -14.9) (width 0.3048) (layer F.Cu) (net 5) (status 10))
 (segment (start 11.5 -18.25) (end 11.25962 -18.49038) (width 0.254) (layer F.Cu) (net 5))
 (segment (start 11.25962 -18.49038) (end 10.25 -18.49038) (width 0.254) (layer F.Cu) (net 5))
 (segment (start 12.325 -18.25) (end 11.5 -18.25) (width 0.254) (layer F.Cu) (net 5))
 (via (at 12.25 -16.5) (size 0.6) (drill 0.4) (layers F.Cu B.Cu) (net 6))
 (segment (start 12.25 -17.175) (end 12.325 -17.25) (width 0.254) (layer F.Cu) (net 6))
 (segment (start 2.25 -16.5) (end 12.25 -16.5) (width 0.254) (layer B.Cu) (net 6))
 (segment (start 12.25 -16.5) (end 12.25 -17.175) (width 0.254) (layer F.Cu) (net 6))
 (segment (start 9.26924 -11.336396) (end 9.26924 -7.48076) (width 0.3048) (layer B.Cu) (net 27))
 (segment (start 9.73076 -7.01924) (end 10.25 -7.01924) (width 0.3048) (layer B.Cu) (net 27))
 (segment (start 9.26924 -7.48076) (end 9.73076 -7.01924) (width 0.3048) (layer B.Cu) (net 27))
 (segment (start 5.705635 -14.9) (end 9.26924 -11.336396) (width 0.3048) (layer B.Cu) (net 27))
 (segment (start 2.25 -14.9) (end 5.705635 -14.9) (width 0.3048) (layer B.Cu) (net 27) (status 10))
 (segment (start 14.175 -17.25) (end 15.75 -17.25) (width 0.254) (layer F.Cu) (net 1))
 (via (at 15.75 -19.5) (size 0.6) (drill 0.4) (layers F.Cu B.Cu) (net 2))
 (segment (start 12.377962 -15.7) (end 15.75 -19.072038) (width 0.254) (layer B.Cu) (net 2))
 (segment (start 15.75 -19.072038) (end 15.75 -19.5) (width 0.254) (layer B.Cu) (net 2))
 (segment (start 2.25 -15.7) (end 12.377962 -15.7) (width 0.254) (layer B.Cu) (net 2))
 (segment (start 15.75 -19.5) (end 15.75 -18.75) (width 0.254) (layer F.Cu) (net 2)))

